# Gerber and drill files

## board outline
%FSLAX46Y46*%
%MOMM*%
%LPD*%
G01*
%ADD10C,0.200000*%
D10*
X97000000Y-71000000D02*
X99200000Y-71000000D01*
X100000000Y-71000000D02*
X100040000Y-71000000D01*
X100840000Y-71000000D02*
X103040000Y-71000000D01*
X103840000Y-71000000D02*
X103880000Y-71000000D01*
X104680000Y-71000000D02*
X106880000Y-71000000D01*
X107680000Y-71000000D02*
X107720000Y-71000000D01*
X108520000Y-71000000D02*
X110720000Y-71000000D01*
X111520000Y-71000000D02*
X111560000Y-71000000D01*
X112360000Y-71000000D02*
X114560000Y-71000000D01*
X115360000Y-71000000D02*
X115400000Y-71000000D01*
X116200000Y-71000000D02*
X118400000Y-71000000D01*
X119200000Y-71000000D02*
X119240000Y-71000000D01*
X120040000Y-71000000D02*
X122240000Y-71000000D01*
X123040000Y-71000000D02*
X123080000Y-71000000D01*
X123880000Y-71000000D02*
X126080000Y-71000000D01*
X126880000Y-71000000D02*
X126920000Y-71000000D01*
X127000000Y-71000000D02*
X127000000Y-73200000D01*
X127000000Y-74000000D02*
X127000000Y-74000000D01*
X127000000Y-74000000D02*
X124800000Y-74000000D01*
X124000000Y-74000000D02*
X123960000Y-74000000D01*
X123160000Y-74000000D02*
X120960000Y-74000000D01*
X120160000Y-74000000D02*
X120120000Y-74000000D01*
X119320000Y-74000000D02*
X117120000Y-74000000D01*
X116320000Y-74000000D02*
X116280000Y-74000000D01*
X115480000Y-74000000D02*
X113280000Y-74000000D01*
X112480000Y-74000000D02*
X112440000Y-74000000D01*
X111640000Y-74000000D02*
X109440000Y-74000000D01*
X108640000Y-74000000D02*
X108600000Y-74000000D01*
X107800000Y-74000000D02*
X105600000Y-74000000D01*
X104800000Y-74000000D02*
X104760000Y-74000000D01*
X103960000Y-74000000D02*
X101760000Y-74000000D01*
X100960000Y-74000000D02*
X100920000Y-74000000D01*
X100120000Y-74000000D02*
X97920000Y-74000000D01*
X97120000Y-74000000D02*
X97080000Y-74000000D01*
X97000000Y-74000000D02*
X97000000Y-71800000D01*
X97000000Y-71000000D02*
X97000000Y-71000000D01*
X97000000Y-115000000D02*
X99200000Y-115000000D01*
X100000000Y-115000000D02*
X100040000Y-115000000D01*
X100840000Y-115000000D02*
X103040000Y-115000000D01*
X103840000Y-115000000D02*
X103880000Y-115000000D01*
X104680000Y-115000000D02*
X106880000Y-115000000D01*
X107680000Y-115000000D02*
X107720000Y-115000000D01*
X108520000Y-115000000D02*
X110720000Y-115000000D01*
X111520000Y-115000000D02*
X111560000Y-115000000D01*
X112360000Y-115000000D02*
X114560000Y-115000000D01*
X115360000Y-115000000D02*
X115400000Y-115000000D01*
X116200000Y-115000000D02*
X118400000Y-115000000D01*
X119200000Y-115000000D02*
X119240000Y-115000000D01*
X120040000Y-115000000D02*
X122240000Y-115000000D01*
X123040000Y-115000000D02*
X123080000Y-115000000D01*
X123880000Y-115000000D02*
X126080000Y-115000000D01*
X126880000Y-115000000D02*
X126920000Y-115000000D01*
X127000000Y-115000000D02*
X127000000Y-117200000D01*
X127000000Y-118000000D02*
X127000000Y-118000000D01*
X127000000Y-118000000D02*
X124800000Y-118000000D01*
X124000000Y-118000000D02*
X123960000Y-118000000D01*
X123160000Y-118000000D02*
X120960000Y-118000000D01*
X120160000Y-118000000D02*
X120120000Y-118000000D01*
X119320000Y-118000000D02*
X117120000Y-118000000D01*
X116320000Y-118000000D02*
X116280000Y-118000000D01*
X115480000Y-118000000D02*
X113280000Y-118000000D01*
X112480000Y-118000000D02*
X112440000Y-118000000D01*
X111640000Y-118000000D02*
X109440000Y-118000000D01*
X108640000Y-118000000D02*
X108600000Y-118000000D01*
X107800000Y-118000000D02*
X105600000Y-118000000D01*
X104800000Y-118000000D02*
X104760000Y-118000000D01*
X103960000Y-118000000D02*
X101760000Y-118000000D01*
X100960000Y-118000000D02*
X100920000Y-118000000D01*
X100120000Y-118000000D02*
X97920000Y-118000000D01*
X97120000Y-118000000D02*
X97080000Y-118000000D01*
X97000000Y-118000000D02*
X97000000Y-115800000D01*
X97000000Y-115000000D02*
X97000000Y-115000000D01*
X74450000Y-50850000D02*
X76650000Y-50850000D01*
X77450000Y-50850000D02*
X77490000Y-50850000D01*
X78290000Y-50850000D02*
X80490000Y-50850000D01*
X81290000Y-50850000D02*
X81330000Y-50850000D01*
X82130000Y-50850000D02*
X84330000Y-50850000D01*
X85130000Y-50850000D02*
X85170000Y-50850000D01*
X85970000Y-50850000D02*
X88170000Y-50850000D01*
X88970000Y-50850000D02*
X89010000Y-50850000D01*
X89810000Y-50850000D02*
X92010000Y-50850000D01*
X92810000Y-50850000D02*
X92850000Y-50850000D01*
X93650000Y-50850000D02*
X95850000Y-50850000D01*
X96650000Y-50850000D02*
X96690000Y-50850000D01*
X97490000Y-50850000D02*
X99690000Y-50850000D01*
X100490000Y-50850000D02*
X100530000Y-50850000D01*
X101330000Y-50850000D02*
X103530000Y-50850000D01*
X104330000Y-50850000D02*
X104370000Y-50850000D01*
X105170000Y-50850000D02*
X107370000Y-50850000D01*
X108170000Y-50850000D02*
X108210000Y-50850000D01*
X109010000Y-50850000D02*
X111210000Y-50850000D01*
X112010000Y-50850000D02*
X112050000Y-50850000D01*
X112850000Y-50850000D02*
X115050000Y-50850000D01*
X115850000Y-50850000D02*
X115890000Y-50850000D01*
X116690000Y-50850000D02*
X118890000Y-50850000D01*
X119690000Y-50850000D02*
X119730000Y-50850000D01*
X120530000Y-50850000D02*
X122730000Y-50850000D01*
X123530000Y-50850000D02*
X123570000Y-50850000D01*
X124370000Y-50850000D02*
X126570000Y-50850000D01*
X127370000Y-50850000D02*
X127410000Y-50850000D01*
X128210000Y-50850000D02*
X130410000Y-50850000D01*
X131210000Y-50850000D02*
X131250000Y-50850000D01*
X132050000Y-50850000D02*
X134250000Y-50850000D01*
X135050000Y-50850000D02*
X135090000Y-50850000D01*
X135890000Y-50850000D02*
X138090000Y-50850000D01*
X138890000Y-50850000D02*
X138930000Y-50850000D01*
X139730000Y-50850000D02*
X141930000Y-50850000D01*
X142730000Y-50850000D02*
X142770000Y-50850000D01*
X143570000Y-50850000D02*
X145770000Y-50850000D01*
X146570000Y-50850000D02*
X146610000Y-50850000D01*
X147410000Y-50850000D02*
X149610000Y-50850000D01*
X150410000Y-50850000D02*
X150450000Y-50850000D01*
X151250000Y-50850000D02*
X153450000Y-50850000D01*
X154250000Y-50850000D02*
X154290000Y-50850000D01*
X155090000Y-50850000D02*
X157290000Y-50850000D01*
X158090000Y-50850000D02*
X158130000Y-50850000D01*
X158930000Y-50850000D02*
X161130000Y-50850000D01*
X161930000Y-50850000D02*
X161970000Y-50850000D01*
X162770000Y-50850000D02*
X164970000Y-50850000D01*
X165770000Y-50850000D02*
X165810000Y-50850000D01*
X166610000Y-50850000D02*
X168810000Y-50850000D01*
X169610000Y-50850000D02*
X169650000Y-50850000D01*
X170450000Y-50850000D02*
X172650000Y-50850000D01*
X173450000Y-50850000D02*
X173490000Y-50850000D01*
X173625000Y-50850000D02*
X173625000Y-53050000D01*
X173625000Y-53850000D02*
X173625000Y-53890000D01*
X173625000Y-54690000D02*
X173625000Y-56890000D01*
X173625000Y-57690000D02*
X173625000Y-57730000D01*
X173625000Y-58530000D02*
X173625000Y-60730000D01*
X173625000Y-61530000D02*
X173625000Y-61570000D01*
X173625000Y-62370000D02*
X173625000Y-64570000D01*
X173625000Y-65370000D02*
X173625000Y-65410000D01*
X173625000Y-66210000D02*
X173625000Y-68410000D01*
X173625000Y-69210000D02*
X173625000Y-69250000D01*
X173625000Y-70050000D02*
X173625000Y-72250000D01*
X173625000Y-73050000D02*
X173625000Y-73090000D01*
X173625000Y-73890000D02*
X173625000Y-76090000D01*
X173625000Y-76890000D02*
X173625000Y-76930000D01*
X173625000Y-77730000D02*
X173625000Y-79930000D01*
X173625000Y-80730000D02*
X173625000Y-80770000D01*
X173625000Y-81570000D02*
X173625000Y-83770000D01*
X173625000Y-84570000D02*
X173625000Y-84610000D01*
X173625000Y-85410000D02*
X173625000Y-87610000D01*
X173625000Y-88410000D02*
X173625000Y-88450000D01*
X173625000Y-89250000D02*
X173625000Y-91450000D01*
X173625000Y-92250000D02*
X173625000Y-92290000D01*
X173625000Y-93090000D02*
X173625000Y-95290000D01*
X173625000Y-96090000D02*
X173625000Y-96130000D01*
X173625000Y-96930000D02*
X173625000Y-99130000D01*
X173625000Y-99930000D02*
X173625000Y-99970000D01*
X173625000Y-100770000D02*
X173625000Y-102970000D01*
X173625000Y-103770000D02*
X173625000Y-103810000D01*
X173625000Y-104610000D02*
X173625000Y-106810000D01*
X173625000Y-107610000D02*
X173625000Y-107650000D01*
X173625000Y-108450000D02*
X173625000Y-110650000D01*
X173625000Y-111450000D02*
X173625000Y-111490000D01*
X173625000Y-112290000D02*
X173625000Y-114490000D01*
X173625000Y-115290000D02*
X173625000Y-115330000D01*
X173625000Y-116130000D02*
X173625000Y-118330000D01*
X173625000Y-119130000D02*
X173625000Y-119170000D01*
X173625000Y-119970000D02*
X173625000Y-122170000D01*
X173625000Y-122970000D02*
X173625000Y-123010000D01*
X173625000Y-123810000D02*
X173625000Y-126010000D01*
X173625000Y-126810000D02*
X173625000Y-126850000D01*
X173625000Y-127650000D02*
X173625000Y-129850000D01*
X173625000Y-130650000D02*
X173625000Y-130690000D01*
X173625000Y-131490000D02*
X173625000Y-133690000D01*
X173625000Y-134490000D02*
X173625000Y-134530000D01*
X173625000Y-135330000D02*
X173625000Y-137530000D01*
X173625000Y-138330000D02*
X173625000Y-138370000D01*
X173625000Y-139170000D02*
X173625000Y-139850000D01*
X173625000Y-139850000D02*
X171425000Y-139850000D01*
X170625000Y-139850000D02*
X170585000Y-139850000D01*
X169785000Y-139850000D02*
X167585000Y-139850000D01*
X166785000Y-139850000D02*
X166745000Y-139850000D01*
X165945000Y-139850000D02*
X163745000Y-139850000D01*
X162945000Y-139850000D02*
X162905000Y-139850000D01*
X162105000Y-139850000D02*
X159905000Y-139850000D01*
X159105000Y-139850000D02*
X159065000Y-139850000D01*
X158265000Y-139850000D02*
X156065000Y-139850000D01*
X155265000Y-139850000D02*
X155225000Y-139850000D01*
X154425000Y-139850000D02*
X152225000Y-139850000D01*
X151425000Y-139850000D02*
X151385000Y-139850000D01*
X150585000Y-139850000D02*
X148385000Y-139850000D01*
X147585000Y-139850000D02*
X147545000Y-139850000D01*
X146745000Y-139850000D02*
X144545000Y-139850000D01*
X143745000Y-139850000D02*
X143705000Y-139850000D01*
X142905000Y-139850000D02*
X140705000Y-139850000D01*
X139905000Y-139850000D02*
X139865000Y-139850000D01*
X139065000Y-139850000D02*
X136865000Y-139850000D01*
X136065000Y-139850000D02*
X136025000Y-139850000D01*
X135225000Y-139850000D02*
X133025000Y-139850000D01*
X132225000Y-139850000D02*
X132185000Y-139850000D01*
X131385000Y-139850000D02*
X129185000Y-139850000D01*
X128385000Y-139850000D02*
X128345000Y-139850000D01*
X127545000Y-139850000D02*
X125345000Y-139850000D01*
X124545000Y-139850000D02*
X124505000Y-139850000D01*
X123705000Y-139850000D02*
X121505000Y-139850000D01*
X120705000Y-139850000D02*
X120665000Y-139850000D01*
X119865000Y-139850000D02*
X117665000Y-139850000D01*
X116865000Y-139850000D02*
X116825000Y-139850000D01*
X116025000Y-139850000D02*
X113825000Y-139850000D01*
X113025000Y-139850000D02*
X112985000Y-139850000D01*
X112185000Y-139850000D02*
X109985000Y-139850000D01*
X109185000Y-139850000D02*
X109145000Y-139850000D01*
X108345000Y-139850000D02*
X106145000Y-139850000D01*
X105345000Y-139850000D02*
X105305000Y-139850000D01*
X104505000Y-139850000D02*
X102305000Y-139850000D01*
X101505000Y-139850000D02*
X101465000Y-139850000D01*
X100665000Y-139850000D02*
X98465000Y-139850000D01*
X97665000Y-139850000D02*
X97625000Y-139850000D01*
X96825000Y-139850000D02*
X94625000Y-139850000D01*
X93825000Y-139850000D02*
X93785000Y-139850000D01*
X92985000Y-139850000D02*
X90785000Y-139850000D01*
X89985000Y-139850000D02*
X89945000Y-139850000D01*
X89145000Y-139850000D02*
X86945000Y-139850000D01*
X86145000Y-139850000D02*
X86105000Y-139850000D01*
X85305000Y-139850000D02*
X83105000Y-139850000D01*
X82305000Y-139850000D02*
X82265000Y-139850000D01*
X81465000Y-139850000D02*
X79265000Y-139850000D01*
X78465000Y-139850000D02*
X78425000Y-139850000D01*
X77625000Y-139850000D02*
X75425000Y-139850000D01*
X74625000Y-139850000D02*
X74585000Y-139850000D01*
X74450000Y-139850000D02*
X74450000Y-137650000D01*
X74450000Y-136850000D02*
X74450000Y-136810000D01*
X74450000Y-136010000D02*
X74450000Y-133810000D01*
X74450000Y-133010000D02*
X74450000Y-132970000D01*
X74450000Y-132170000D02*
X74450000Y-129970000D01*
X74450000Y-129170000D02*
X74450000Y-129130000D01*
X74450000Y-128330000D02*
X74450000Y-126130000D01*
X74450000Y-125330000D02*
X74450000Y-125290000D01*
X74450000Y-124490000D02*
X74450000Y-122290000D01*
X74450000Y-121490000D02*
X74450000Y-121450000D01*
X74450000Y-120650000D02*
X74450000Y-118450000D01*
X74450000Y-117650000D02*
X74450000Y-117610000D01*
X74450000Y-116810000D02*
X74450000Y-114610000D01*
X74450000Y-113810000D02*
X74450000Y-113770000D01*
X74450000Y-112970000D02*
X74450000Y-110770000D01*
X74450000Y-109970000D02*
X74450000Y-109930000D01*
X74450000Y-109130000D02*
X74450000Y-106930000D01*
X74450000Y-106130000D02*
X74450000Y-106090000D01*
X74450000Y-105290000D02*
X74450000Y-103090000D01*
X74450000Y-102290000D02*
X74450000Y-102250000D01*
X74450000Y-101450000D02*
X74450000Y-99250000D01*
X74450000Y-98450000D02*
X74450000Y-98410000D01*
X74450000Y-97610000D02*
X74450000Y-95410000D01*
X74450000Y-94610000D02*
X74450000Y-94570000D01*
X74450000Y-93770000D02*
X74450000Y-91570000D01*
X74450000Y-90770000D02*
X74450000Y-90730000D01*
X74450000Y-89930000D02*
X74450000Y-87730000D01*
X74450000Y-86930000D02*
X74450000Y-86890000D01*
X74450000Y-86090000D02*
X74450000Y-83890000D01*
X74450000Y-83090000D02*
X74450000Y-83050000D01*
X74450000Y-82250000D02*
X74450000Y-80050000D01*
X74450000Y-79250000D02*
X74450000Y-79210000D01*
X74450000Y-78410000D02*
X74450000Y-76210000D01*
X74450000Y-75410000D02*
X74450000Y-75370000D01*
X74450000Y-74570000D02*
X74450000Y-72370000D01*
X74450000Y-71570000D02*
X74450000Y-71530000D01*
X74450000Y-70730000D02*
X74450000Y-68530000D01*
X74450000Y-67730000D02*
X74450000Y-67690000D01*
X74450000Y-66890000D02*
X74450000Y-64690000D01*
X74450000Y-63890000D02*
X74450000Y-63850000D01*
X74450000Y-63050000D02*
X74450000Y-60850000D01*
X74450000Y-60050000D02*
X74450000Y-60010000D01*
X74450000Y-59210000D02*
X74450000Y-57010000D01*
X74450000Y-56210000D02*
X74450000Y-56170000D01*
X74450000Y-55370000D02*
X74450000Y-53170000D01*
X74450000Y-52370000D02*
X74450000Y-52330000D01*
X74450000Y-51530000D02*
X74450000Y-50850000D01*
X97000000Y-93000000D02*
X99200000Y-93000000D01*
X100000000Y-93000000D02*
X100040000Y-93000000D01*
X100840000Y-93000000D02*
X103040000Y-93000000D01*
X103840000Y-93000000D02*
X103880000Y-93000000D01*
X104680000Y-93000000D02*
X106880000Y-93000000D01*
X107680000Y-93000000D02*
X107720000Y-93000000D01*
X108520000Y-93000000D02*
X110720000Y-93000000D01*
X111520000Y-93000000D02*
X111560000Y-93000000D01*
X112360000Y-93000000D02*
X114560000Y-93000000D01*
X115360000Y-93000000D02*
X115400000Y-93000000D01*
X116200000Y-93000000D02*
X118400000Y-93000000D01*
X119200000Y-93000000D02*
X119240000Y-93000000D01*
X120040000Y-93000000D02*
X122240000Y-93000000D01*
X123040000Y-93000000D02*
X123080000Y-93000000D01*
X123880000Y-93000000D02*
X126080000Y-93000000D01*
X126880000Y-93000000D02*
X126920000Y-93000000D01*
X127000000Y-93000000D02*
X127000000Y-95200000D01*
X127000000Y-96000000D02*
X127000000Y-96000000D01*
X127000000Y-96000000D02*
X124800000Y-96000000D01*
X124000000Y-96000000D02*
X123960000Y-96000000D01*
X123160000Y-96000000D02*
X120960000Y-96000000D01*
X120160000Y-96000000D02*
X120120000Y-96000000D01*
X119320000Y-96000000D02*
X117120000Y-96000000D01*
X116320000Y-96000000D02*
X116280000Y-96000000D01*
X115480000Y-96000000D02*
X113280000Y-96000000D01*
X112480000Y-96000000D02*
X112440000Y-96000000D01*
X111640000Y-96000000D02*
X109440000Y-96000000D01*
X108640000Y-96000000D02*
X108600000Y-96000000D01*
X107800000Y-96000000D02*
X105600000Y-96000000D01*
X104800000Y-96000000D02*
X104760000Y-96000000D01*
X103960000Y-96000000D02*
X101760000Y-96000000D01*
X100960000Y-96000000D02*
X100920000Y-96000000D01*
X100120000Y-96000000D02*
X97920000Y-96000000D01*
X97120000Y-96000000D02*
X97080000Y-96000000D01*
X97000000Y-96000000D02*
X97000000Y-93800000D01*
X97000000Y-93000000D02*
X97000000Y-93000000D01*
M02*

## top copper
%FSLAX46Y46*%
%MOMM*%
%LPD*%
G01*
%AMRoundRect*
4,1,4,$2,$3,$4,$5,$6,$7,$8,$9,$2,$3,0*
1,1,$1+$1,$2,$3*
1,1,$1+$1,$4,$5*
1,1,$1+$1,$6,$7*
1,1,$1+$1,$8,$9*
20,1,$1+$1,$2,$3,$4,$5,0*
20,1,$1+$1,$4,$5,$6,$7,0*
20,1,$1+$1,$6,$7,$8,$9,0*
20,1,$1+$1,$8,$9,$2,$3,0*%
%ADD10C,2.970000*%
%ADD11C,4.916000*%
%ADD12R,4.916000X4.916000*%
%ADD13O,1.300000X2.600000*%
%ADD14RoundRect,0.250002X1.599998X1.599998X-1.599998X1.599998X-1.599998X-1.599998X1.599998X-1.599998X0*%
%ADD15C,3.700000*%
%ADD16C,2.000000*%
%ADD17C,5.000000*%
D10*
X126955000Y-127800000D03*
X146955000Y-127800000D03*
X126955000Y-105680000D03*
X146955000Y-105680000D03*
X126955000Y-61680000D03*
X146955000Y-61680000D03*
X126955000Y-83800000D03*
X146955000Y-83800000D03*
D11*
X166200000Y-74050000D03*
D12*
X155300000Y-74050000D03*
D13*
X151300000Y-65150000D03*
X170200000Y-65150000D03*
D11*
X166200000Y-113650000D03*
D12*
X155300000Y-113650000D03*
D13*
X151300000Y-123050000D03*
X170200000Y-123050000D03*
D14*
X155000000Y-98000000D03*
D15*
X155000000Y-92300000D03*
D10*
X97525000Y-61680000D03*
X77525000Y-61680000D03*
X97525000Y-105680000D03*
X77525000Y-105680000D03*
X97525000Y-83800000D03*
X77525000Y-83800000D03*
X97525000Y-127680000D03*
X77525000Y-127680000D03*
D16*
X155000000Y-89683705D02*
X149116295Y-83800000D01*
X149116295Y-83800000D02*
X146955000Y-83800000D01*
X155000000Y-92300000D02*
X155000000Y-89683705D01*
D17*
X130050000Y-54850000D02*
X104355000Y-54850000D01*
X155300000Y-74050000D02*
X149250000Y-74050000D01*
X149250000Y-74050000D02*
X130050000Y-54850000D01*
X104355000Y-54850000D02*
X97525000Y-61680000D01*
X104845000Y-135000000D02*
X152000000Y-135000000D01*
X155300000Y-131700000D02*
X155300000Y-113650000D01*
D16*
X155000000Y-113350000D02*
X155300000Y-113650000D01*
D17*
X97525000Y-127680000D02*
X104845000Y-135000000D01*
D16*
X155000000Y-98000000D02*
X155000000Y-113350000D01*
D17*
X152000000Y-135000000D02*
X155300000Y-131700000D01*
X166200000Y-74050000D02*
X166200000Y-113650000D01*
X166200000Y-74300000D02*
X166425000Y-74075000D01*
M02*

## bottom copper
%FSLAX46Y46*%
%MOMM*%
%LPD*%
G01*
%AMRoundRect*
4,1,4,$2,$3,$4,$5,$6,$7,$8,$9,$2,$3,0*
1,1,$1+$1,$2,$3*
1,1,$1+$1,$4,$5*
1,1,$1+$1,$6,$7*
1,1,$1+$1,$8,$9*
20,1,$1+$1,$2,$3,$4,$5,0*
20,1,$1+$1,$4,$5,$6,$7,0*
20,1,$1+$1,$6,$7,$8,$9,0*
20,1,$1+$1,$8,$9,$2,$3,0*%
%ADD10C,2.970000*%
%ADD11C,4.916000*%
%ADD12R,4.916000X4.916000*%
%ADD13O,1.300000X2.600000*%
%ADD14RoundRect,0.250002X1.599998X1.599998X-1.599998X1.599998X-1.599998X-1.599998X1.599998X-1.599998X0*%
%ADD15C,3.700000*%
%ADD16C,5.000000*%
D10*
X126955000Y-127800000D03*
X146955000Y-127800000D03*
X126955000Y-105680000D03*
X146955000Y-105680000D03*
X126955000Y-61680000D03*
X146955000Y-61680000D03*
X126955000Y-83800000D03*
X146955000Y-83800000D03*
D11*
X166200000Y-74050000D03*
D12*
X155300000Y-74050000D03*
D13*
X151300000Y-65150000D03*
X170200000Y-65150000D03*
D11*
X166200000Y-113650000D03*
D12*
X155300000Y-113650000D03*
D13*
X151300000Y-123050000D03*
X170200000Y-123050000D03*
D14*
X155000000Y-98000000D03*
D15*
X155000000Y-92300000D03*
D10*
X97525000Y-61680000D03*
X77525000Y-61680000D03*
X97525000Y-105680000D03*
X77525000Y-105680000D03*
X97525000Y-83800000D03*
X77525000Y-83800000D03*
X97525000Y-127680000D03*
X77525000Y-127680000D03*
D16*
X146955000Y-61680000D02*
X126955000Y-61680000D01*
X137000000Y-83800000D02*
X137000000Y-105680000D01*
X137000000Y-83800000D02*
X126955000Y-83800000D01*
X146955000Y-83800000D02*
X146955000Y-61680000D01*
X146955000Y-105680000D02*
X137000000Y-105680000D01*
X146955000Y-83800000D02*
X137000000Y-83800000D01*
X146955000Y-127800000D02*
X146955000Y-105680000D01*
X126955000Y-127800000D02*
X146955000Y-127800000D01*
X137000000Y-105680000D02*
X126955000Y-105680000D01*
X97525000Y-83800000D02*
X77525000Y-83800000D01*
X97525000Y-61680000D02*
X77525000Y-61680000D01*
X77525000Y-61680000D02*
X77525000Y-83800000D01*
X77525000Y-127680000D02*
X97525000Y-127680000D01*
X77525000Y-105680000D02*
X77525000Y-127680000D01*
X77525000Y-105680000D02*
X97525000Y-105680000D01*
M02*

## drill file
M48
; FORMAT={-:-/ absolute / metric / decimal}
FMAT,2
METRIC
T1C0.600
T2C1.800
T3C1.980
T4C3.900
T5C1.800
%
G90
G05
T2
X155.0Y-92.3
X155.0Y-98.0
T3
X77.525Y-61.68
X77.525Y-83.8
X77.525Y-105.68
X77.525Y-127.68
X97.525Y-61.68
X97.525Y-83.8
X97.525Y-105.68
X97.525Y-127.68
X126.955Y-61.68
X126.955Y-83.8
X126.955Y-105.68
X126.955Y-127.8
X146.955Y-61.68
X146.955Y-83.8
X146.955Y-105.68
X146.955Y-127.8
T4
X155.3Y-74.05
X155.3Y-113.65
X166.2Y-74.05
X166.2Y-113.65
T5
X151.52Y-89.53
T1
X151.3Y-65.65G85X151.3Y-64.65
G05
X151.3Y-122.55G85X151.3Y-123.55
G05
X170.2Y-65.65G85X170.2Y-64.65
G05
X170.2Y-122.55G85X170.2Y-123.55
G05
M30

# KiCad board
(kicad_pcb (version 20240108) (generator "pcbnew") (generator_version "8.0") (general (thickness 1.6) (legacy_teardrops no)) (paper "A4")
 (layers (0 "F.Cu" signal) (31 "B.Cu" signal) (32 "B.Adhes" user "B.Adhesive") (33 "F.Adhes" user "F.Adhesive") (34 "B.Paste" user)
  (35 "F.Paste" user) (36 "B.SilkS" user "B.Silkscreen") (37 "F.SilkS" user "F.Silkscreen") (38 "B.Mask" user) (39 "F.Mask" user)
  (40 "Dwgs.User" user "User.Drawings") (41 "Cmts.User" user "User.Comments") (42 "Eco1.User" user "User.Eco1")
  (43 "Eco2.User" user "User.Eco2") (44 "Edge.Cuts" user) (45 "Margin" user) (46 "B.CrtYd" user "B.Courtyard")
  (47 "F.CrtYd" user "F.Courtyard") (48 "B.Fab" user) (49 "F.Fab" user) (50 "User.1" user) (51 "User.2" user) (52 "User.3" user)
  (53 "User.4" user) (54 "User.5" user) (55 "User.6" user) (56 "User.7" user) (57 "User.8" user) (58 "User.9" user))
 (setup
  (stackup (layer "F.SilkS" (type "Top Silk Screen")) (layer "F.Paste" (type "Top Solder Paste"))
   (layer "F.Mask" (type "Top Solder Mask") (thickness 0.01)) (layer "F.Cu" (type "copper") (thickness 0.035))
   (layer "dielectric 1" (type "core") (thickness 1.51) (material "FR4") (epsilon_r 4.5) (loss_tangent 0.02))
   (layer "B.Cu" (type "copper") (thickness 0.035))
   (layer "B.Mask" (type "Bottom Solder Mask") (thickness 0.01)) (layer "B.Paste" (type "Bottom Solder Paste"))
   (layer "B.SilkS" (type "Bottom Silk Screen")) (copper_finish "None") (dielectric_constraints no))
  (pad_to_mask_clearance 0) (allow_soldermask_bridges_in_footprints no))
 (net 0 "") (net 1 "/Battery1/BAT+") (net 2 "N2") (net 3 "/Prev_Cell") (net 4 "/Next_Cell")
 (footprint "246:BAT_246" (layer "F.Cu") (at 136.955 127.8)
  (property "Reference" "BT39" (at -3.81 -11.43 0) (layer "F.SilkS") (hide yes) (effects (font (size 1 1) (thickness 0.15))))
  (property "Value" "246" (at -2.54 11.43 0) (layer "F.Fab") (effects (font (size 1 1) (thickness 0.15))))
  (pad "A" thru_hole circle (at -10 0) (size 2.97 2.97) (drill 1.98) (layers "*.Cu") (remove_unused_layers no) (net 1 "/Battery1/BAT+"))
  (pad "A" thru_hole circle (at 10 0) (size 2.97 2.97) (drill 1.98) (layers "*.Cu") (remove_unused_layers no) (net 1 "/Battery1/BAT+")))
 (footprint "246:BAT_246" (layer "F.Cu") (at 136.955 105.68)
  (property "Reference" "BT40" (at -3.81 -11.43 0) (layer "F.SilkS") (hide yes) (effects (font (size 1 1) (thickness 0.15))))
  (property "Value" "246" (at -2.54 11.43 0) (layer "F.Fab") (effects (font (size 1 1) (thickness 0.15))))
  (pad "A" thru_hole circle (at -10 0) (size 2.97 2.97) (drill 1.98) (layers "*.Cu") (remove_unused_layers no) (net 1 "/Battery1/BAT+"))
  (pad "A" thru_hole circle (at 10 0) (size 2.97 2.97) (drill 1.98) (layers "*.Cu") (remove_unused_layers no) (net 1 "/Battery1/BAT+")))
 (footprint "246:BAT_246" (layer "F.Cu") (at 136.955 61.68)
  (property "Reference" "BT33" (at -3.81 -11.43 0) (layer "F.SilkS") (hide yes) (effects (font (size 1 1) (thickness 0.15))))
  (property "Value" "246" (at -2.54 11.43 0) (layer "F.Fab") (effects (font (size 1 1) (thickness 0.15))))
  (pad "A" thru_hole circle (at -10 0) (size 2.97 2.97) (drill 1.98) (layers "*.Cu") (remove_unused_layers no) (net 1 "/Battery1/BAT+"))
  (pad "A" thru_hole circle (at 10 0) (size 2.97 2.97) (drill 1.98) (layers "*.Cu") (remove_unused_layers no) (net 1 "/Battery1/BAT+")))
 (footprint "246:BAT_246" (layer "F.Cu") (at 136.955 83.8)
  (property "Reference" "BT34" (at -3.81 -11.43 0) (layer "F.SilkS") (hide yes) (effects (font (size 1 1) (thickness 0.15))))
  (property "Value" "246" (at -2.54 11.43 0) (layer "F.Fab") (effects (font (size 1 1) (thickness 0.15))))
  (pad "A" thru_hole circle (at -10 0) (size 2.97 2.97) (drill 1.98) (layers "*.Cu") (remove_unused_layers no) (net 1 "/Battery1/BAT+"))
  (pad "A" thru_hole circle (at 10 0) (size 2.97 2.97) (drill 1.98) (layers "*.Cu") (remove_unused_layers no) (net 1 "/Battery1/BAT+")))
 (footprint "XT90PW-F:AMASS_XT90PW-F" (layer "F.Cu") (at 160.75 65.15 180)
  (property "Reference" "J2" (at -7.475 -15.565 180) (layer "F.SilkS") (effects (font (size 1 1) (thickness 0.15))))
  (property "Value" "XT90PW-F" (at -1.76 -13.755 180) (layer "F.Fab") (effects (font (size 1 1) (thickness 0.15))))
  (pad "N" thru_hole circle (at -5.45 -8.9 180) (size 4.916 4.916) (drill 3.9) (layers "*.Cu" "*.Mask") (remove_unused_layers no)
   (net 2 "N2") (solder_mask_margin 0.102))
  (pad "P" thru_hole rect (at 5.45 -8.9 180) (size 4.916 4.916) (drill 3.9) (layers "*.Cu" "*.Mask") (remove_unused_layers no)
   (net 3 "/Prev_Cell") (solder_mask_margin 0.102))
  (pad "S1" thru_hole oval (at 9.45 0 180) (size 1.3 2.6) (drill oval 0.6 1.6) (layers "*.Cu" "*.Mask") (remove_unused_layers no)
   (solder_mask_margin 0.102))
  (pad "S2" thru_hole oval (at -9.45 0 180) (size 1.3 2.6) (drill oval 0.6 1.6) (layers "*.Cu" "*.Mask") (remove_unused_layers no)
   (solder_mask_margin 0.102)))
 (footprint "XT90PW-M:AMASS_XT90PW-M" (layer "F.Cu") (at 160.75 123.05)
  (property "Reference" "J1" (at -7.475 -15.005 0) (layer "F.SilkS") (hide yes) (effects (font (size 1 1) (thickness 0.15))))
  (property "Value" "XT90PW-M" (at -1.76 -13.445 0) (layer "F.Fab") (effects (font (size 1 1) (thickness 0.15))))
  (pad "N" thru_hole circle (at 5.45 -9.4) (size 4.916 4.916) (drill 3.9) (layers "*.Cu" "*.Mask") (remove_unused_layers no) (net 2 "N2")
   (solder_mask_margin 0.102))
  (pad "P" thru_hole rect (at -5.45 -9.4) (size 4.916 4.916) (drill 3.9) (layers "*.Cu" "*.Mask") (remove_unused_layers no)
   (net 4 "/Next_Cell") (solder_mask_margin 0.102))
  (pad "S1" thru_hole oval (at -9.45 0) (size 1.3 2.6) (drill oval 0.6 1.6) (layers "*.Cu" "*.Mask") (remove_unused_layers no)
   (solder_mask_margin 0.102))
  (pad "S2" thru_hole oval (at 9.45 0) (size 1.3 2.6) (drill oval 0.6 1.6) (layers "*.Cu" "*.Mask") (remove_unused_layers no)
   (solder_mask_margin 0.102)))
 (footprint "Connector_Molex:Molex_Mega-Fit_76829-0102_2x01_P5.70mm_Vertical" (layer "F.Cu") (at 155 98 180)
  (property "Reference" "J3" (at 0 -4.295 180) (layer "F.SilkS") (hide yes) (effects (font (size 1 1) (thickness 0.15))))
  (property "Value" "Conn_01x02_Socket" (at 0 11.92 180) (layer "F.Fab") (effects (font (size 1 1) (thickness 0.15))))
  (pad "" np_thru_hole circle (at 3.48 8.47 180) (size 1.8 1.8) (drill 1.8) (layers "*.Cu" "*.Mask"))
  (pad "1" thru_hole roundrect (at 0 0 180) (size 3.7 3.7) (drill 1.8) (layers "*.Cu" "*.Mask") (remove_unused_layers no)
   (roundrect_rratio 0.067568) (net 4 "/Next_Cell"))
  (pad "2" thru_hole circle (at 0 5.7 180) (size 3.7 3.7) (drill 1.8) (layers "*.Cu" "*.Mask") (remove_unused_layers no)
   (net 1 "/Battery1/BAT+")))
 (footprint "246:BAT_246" (layer "F.Cu") (at 87.525 61.68 180)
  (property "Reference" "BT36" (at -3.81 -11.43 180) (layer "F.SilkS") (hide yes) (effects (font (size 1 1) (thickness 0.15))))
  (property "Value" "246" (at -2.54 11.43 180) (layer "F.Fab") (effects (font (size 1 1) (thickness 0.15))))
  (pad "A" thru_hole circle (at -10 0 180) (size 2.97 2.97) (drill 1.98) (layers "*.Cu") (remove_unused_layers no) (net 3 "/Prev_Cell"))
  (pad "A" thru_hole circle (at 10 0 180) (size 2.97 2.97) (drill 1.98) (layers "*.Cu") (remove_unused_layers no) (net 3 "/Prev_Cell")))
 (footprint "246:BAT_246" (layer "F.Cu") (at 87.525 105.68 180)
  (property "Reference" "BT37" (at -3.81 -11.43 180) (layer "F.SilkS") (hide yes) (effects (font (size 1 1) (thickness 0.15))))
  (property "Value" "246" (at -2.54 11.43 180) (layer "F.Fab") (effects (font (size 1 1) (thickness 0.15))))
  (pad "A" thru_hole circle (at -10 0 180) (size 2.97 2.97) (drill 1.98) (layers "*.Cu") (remove_unused_layers no) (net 4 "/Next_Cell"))
  (pad "A" thru_hole circle (at 10 0 180) (size 2.97 2.97) (drill 1.98) (layers "*.Cu") (remove_unused_layers no) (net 4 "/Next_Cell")))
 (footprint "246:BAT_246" (layer "F.Cu") (at 87.525 83.8 180)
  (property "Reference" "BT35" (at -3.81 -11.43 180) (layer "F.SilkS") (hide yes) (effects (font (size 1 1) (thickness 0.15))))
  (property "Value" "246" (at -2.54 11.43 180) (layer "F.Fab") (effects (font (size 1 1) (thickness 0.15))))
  (pad "A" thru_hole circle (at -10 0 180) (size 2.97 2.97) (drill 1.98) (layers "*.Cu") (remove_unused_layers no) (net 3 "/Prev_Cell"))
  (pad "A" thru_hole circle (at 10 0 180) (size 2.97 2.97) (drill 1.98) (layers "*.Cu") (remove_unused_layers no) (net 3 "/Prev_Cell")))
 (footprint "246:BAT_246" (layer "F.Cu") (at 87.525 127.68 180)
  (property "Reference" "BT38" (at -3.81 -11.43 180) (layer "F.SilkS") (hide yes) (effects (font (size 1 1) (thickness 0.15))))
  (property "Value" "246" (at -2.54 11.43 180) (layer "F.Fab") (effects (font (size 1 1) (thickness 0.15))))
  (pad "A" thru_hole circle (at -10 0 180) (size 2.97 2.97) (drill 1.98) (layers "*.Cu") (remove_unused_layers no) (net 4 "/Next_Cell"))
  (pad "A" thru_hole circle (at 10 0 180) (size 2.97 2.97) (drill 1.98) (layers "*.Cu") (remove_unused_layers no) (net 4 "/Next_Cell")))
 (gr_rect (start 97 71) (end 127 74) (stroke (width 0.2) (type dash_dot)) (fill none) (layer "Edge.Cuts"))
 (gr_rect (start 97 115) (end 127 118) (stroke (width 0.2) (type dash_dot)) (fill none) (layer "Edge.Cuts"))
 (gr_rect (start 74.45 50.85) (end 173.625 139.85) (stroke (width 0.2) (type dash_dot)) (fill none) (layer "Edge.Cuts"))
 (gr_rect (start 97 93) (end 127 96) (stroke (width 0.2) (type dash_dot)) (fill none) (layer "Edge.Cuts"))
 (segment (start 155 89.683705) (end 149.116295 83.8) (width 2) (layer "F.Cu") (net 1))
 (segment (start 149.116295 83.8) (end 146.955 83.8) (width 2) (layer "F.Cu") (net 1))
 (segment (start 155 92.3) (end 155 89.683705) (width 2) (layer "F.Cu") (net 1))
 (segment (start 146.955 61.68) (end 126.955 61.68) (width 5) (layer "B.Cu") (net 1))
 (segment (start 137 83.8) (end 137 105.68) (width 5) (layer "B.Cu") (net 1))
 (segment (start 137 83.8) (end 126.955 83.8) (width 5) (layer "B.Cu") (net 1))
 (segment (start 146.955 83.8) (end 146.955 61.68) (width 5) (layer "B.Cu") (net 1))
 (segment (start 146.955 105.68) (end 137 105.68) (width 5) (layer "B.Cu") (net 1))
 (segment (start 146.955 83.8) (end 137 83.8) (width 5) (layer "B.Cu") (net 1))
 (segment (start 146.955 127.8) (end 146.955 105.68) (width 5) (layer "B.Cu") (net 1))
 (segment (start 126.955 127.8) (end 146.955 127.8) (width 5) (layer "B.Cu") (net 1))
 (segment (start 137 105.68) (end 126.955 105.68) (width 5) (layer "B.Cu") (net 1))
 (segment (start 130.05 54.85) (end 104.355 54.85) (width 5) (layer "F.Cu") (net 3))
 (segment (start 155.3 74.05) (end 149.25 74.05) (width 5) (layer "F.Cu") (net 3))
 (segment (start 149.25 74.05) (end 130.05 54.85) (width 5) (layer "F.Cu") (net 3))
 (segment (start 104.355 54.85) (end 97.525 61.68) (width 5) (layer "F.Cu") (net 3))
 (segment (start 97.525 83.8) (end 77.525 83.8) (width 5) (layer "B.Cu") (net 3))
 (segment (start 97.525 61.68) (end 77.525 61.68) (width 5) (layer "B.Cu") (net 3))
 (segment (start 77.525 61.68) (end 77.525 83.8) (width 5) (layer "B.Cu") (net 3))
 (segment (start 104.845 135) (end 152 135) (width 5) (layer "F.Cu") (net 4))
 (segment (start 155.3 131.7) (end 155.3 113.65) (width 5) (layer "F.Cu") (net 4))
 (segment (start 155 113.35) (end 155.3 113.65) (width 2) (layer "F.Cu") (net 4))
 (segment (start 97.525 127.68) (end 104.845 135) (width 5) (layer "F.Cu") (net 4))
 (segment (start 155 98) (end 155 113.35) (width 2) (layer "F.Cu") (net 4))
 (segment (start 152 135) (end 155.3 131.7) (width 5) (layer "F.Cu") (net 4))
 (segment (start 77.525 127.68) (end 97.525 127.68) (width 5) (layer "B.Cu") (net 4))
 (segment (start 77.525 105.68) (end 77.525 127.68) (width 5) (layer "B.Cu") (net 4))
 (segment (start 77.525 105.68) (end 97.525 105.68) (width 5) (layer "B.Cu") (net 4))
 (segment (start 166.2 74.05) (end 166.2 113.65) (width 5) (layer "F.Cu") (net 2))
 (segment (start 166.2 74.3) (end 166.425 74.075) (width 5) (layer "F.Cu") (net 2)))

